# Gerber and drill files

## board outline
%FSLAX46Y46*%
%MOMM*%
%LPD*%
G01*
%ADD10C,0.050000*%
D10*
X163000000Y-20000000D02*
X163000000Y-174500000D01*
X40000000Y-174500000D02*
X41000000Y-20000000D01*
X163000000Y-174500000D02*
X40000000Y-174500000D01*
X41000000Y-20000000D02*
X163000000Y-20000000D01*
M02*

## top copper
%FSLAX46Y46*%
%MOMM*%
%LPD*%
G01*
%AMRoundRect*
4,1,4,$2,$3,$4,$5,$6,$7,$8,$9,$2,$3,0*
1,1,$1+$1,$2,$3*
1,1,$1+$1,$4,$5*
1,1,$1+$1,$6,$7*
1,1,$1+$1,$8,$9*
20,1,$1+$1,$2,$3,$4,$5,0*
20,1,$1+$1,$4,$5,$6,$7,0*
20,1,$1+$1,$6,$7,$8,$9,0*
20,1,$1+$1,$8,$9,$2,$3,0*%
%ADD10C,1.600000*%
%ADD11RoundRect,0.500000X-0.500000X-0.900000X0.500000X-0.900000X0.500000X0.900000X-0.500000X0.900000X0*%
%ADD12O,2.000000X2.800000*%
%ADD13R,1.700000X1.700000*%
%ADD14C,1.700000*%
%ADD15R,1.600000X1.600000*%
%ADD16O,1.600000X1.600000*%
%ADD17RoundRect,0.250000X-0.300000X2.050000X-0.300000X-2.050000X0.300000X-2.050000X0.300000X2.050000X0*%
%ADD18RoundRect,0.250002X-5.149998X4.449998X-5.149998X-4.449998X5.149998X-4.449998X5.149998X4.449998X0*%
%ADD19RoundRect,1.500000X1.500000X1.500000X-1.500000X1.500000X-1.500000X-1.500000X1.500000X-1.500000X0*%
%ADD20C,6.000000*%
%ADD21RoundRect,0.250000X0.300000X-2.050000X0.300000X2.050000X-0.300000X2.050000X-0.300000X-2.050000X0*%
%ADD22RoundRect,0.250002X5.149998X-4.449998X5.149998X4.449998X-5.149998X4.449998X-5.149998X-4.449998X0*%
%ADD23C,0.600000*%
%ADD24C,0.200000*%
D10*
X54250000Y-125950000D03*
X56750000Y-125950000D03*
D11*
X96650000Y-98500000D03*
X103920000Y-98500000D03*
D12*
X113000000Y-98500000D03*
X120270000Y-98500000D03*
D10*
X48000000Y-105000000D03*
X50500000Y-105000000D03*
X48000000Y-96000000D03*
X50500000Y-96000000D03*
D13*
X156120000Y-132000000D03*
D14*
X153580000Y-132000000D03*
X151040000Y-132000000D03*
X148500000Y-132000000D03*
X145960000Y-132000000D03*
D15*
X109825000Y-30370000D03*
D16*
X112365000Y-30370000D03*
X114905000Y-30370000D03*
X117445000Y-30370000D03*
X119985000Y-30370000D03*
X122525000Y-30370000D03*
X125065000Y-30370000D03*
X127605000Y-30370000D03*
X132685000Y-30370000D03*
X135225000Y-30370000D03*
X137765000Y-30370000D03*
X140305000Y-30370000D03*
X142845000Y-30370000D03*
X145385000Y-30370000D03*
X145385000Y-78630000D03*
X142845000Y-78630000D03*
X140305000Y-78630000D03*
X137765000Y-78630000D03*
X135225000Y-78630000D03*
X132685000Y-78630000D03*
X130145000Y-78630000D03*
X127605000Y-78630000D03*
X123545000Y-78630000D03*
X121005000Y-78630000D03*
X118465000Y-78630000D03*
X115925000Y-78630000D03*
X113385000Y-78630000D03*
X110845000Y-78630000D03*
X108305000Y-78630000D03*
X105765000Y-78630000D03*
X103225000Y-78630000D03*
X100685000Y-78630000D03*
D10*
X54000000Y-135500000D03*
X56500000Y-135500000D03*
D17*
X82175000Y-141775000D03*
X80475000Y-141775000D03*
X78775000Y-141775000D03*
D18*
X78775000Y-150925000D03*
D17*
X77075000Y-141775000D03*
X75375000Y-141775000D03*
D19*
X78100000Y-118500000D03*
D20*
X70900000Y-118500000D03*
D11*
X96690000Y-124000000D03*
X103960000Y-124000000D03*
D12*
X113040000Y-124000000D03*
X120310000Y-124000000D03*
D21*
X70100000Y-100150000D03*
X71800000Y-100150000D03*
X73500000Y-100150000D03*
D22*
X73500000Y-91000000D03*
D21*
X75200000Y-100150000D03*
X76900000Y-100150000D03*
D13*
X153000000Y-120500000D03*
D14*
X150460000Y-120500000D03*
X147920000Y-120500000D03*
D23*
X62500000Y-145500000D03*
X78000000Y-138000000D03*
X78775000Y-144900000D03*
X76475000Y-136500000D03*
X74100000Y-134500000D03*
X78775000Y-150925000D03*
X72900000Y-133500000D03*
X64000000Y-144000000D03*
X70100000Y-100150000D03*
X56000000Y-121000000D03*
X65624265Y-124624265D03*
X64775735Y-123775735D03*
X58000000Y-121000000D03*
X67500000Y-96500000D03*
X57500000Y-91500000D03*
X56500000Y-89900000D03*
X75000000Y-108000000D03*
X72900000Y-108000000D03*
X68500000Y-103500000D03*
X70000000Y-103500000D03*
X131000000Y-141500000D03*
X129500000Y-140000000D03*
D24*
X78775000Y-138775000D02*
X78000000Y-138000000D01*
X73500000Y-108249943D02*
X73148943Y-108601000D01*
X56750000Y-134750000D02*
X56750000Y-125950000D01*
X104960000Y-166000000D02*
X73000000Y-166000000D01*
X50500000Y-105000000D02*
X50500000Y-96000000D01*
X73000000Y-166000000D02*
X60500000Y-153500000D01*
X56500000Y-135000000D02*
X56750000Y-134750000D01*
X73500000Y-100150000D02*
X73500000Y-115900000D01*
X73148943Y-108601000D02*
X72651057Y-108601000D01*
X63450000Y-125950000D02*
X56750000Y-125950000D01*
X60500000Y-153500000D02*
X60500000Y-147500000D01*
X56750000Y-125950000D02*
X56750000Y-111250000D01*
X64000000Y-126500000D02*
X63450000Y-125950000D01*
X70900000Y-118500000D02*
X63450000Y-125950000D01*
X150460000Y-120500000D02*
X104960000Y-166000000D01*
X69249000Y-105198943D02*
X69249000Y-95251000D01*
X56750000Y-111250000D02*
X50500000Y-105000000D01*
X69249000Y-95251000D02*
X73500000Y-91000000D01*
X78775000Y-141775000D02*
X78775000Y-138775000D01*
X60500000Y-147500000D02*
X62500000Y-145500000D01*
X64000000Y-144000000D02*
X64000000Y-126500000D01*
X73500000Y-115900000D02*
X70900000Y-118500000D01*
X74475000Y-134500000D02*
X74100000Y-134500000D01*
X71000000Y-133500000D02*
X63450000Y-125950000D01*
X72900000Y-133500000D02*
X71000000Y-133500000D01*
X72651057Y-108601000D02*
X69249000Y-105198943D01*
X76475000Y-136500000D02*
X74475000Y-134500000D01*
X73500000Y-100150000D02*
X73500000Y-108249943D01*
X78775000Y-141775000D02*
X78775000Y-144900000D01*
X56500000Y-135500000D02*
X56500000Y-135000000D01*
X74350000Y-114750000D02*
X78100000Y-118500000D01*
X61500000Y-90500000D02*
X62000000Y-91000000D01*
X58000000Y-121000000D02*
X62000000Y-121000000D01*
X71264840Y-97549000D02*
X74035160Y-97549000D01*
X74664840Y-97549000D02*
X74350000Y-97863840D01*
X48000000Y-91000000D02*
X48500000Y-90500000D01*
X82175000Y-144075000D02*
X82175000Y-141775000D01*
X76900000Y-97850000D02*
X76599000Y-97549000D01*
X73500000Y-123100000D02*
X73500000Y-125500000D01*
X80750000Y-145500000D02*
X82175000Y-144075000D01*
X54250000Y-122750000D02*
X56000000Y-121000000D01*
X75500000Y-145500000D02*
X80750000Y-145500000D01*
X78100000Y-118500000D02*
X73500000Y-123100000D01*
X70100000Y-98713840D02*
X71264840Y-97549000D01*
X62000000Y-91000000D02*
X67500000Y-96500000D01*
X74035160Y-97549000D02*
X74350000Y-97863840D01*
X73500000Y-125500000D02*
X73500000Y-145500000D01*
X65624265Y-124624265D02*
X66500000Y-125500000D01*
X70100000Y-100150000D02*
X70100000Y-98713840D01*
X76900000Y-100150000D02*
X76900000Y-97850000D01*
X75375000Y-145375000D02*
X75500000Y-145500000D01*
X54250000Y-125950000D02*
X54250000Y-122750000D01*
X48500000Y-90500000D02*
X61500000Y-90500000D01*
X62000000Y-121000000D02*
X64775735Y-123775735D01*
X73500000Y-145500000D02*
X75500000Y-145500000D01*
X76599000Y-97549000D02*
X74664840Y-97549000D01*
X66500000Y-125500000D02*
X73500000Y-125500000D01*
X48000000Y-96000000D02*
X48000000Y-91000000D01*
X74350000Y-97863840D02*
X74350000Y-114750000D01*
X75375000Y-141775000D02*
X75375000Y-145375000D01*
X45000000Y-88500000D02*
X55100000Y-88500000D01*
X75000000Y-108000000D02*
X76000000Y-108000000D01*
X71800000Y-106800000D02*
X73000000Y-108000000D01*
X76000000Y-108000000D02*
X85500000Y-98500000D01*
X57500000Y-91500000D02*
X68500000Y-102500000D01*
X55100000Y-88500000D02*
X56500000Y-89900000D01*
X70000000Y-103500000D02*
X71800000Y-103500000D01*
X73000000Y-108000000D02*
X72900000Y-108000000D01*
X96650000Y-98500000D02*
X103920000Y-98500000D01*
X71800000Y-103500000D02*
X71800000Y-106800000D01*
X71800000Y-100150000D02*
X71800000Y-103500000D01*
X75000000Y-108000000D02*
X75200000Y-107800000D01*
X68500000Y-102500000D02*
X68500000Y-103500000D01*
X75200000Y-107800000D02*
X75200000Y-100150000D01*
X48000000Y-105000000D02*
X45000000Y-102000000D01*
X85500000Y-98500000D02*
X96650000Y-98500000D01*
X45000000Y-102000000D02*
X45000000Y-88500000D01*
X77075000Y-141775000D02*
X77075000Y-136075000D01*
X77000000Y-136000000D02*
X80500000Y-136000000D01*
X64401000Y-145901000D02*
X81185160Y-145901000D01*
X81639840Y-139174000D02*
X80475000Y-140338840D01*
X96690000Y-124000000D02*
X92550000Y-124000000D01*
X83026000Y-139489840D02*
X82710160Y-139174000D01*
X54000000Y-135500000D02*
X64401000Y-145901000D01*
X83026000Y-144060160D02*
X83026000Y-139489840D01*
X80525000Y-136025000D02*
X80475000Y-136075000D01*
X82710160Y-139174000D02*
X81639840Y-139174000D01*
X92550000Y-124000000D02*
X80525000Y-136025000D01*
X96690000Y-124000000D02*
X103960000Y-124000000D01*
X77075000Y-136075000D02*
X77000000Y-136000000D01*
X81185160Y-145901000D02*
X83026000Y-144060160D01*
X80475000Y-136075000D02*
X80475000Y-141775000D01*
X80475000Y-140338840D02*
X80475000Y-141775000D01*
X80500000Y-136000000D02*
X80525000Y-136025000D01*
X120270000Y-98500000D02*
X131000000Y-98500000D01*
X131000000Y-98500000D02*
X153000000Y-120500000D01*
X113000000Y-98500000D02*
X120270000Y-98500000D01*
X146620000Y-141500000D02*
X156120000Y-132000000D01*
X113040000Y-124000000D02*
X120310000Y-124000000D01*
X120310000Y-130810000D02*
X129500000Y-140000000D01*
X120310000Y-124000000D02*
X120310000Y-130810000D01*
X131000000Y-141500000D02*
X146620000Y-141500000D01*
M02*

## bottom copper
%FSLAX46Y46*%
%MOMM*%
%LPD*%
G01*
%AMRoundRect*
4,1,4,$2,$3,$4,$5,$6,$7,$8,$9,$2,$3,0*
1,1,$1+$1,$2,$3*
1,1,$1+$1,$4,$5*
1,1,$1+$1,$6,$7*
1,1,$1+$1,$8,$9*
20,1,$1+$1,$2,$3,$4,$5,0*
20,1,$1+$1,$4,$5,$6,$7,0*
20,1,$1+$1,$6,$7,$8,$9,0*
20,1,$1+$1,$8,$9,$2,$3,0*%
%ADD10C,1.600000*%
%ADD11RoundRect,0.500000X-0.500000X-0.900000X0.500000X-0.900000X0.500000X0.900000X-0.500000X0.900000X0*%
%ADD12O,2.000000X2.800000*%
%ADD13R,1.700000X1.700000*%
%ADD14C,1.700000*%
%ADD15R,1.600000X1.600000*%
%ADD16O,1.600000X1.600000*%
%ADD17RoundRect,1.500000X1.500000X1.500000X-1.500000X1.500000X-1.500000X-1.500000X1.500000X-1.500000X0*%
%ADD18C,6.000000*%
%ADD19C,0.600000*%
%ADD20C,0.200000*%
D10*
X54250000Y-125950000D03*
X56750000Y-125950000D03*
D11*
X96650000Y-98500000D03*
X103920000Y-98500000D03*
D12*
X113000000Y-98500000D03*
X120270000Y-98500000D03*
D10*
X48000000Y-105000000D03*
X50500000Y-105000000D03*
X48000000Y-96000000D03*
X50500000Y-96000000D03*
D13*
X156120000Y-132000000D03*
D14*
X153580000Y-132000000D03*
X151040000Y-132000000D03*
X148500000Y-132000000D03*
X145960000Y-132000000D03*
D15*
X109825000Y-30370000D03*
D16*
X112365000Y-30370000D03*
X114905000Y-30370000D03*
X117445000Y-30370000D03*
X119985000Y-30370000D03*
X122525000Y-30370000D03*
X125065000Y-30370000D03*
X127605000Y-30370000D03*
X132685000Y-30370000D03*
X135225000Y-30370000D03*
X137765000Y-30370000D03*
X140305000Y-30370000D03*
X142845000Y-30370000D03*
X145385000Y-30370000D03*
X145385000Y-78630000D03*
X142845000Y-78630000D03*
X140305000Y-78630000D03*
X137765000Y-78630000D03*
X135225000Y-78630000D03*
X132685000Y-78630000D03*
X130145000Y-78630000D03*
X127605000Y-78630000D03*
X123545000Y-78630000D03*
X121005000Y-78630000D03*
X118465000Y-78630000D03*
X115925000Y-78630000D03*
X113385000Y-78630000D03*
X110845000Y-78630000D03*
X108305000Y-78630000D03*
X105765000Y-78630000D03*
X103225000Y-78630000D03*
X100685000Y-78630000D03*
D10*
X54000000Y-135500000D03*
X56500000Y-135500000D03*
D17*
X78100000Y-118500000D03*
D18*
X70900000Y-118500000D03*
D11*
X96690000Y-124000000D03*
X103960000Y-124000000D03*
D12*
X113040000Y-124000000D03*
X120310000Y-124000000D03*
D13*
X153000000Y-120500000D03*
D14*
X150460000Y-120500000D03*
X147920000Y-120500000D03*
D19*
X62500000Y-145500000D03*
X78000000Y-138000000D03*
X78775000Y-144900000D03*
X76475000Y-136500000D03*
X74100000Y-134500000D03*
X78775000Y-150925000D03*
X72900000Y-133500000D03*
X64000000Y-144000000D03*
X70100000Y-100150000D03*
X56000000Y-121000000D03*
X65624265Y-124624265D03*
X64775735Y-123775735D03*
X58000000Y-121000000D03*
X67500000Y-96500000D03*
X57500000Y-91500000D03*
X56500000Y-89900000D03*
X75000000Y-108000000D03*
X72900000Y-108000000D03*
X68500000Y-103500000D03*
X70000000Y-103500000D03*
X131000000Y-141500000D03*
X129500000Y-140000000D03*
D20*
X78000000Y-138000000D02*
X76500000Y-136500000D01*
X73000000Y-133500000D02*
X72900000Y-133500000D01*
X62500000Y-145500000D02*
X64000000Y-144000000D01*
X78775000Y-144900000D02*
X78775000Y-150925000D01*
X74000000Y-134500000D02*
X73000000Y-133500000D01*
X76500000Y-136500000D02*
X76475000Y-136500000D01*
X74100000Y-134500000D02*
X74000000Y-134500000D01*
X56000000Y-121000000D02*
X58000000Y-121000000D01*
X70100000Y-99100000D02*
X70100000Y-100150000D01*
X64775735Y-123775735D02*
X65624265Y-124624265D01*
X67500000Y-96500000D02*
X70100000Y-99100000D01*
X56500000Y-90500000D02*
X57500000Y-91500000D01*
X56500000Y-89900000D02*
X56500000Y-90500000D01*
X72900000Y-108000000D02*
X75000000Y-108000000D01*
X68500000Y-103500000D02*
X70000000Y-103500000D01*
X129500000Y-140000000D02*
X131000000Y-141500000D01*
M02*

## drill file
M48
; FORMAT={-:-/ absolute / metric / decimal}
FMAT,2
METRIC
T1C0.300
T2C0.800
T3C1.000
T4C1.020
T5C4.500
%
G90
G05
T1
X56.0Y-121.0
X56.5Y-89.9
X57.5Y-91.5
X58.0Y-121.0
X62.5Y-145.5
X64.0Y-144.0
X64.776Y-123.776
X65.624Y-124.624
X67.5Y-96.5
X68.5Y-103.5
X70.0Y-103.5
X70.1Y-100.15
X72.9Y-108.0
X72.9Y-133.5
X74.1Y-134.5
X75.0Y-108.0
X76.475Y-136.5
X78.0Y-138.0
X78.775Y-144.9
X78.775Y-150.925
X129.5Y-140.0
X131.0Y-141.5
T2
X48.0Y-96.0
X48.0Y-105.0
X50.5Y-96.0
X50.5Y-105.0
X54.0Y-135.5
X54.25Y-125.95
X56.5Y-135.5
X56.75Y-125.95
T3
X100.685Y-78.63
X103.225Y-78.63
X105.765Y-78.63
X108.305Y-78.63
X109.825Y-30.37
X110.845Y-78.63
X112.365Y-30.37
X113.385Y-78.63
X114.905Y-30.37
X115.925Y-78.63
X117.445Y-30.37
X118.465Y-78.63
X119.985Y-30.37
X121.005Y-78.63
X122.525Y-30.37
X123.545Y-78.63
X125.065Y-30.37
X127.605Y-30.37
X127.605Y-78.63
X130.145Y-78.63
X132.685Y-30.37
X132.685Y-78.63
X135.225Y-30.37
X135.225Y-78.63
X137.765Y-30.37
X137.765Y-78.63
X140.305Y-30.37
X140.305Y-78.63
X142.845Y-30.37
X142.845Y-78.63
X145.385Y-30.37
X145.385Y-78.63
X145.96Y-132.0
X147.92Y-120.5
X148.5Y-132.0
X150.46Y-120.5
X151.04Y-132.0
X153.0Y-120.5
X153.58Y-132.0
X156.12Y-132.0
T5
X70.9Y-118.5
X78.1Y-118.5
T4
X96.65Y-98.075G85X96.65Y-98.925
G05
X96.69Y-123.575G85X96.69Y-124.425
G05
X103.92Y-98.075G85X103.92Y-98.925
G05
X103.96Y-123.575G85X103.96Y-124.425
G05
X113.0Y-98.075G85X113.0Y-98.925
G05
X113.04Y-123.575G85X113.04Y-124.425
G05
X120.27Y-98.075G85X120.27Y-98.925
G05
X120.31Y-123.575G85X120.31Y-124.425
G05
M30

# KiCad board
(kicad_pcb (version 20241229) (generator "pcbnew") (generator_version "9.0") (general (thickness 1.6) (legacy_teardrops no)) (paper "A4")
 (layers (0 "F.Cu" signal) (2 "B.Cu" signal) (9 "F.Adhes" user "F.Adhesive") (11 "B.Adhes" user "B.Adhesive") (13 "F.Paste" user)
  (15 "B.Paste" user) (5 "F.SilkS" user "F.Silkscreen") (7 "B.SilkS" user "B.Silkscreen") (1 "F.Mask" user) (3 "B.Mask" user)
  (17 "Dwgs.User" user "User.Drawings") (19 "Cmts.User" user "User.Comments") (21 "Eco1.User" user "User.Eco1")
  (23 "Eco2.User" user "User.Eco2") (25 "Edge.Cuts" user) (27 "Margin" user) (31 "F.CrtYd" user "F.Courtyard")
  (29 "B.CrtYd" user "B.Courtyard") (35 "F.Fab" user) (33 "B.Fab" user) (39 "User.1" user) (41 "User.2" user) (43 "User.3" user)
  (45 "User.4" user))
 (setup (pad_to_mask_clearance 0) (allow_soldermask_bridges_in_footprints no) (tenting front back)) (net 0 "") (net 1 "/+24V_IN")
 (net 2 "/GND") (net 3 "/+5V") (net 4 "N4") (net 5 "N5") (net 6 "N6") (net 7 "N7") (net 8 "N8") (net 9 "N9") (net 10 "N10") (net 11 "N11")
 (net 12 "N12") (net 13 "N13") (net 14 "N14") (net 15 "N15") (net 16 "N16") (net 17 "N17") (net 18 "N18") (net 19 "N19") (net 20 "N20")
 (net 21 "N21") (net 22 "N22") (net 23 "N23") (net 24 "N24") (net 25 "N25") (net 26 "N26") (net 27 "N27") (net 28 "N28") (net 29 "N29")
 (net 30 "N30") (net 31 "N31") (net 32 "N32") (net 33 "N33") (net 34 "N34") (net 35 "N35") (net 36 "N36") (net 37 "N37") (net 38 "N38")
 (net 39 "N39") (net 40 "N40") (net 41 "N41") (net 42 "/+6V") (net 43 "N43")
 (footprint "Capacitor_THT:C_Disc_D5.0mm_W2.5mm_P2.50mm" (layer "F.Cu") (at 54.25 125.95)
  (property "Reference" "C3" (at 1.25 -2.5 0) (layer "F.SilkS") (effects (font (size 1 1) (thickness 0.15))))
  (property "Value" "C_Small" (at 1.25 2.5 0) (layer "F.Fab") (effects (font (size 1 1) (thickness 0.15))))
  (pad "1" thru_hole circle (at 0 0) (size 1.6 1.6) (drill 0.8) (layers "*.Cu" "*.Mask") (remove_unused_layers no) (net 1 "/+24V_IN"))
  (pad "2" thru_hole circle (at 2.5 0) (size 1.6 1.6) (drill 0.8) (layers "*.Cu" "*.Mask") (remove_unused_layers no) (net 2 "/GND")))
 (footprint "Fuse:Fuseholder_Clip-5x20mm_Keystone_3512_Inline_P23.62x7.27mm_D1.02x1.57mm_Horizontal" (layer "F.Cu") (at 96.65 98.5)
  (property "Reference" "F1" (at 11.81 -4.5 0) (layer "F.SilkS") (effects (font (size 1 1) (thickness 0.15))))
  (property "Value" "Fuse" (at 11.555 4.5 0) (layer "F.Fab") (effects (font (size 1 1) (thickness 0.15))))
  (pad "1" thru_hole roundrect (at 0 0) (size 2 2.8) (drill oval 1.02 1.87) (layers "*.Cu" "*.Mask") (remove_unused_layers no)
   (roundrect_rratio 0.25) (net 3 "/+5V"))
  (pad "1" thru_hole roundrect (at 7.27 0) (size 2 2.8) (drill oval 1.02 1.87) (layers "*.Cu" "*.Mask") (remove_unused_layers no)
   (roundrect_rratio 0.25) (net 3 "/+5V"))
  (pad "2" thru_hole oval (at 16.35 0) (size 2 2.8) (drill oval 1.02 1.87) (layers "*.Cu" "*.Mask") (remove_unused_layers no) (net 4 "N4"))
  (pad "2" thru_hole oval (at 23.62 0) (size 2 2.8) (drill oval 1.02 1.87) (layers "*.Cu" "*.Mask") (remove_unused_layers no) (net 4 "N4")))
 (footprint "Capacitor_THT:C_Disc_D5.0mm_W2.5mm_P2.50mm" (layer "F.Cu") (at 48 105)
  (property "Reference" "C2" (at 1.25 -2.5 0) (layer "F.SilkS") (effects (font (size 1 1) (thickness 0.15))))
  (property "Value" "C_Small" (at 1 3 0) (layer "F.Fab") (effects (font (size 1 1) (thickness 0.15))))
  (pad "1" thru_hole circle (at 0 0) (size 1.6 1.6) (drill 0.8) (layers "*.Cu" "*.Mask") (remove_unused_layers no) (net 3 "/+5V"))
  (pad "2" thru_hole circle (at 2.5 0) (size 1.6 1.6) (drill 0.8) (layers "*.Cu" "*.Mask") (remove_unused_layers no) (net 2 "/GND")))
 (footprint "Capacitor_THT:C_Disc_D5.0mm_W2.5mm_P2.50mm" (layer "F.Cu") (at 48 96)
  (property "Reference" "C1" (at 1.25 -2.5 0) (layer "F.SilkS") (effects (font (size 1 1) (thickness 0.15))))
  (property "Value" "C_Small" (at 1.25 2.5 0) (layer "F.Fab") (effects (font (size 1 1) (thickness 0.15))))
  (pad "1" thru_hole circle (at 0 0) (size 1.6 1.6) (drill 0.8) (layers "*.Cu" "*.Mask") (remove_unused_layers no) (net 1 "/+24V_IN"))
  (pad "2" thru_hole circle (at 2.5 0) (size 1.6 1.6) (drill 0.8) (layers "*.Cu" "*.Mask") (remove_unused_layers no) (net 2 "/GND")))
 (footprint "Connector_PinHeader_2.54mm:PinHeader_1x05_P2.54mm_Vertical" (layer "F.Cu") (at 156.12 132 -90)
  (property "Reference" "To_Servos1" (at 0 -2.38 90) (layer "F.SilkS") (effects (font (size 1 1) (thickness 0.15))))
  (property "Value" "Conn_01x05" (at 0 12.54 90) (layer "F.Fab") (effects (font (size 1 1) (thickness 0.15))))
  (pad "1" thru_hole rect (at 0 0 270) (size 1.7 1.7) (drill 1) (layers "*.Cu" "*.Mask") (remove_unused_layers no) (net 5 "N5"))
  (pad "2" thru_hole circle (at 0 2.54 270) (size 1.7 1.7) (drill 1) (layers "*.Cu" "*.Mask") (remove_unused_layers no) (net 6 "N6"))
  (pad "3" thru_hole circle (at 0 5.08 270) (size 1.7 1.7) (drill 1) (layers "*.Cu" "*.Mask") (remove_unused_layers no) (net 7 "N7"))
  (pad "4" thru_hole circle (at 0 7.62 270) (size 1.7 1.7) (drill 1) (layers "*.Cu" "*.Mask") (remove_unused_layers no) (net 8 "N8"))
  (pad "5" thru_hole circle (at 0 10.16 270) (size 1.7 1.7) (drill 1) (layers "*.Cu" "*.Mask") (remove_unused_layers no) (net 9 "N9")))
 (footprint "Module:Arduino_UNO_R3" (layer "F.Cu") (at 109.825 30.37)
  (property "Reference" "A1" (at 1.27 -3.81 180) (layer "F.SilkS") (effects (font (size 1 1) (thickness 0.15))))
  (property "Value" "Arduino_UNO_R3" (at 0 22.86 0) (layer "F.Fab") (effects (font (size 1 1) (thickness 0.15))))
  (pad "1" thru_hole rect (at 0 0 90) (size 1.6 1.6) (drill 1) (layers "*.Cu" "*.Mask") (remove_unused_layers no) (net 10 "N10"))
  (pad "2" thru_hole oval (at 2.54 0 90) (size 1.6 1.6) (drill 1) (layers "*.Cu" "*.Mask") (remove_unused_layers no) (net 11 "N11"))
  (pad "3" thru_hole oval (at 5.08 0 90) (size 1.6 1.6) (drill 1) (layers "*.Cu" "*.Mask") (remove_unused_layers no) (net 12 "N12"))
  (pad "4" thru_hole oval (at 7.62 0 90) (size 1.6 1.6) (drill 1) (layers "*.Cu" "*.Mask") (remove_unused_layers no) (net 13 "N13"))
  (pad "5" thru_hole oval (at 10.16 0 90) (size 1.6 1.6) (drill 1) (layers "*.Cu" "*.Mask") (remove_unused_layers no) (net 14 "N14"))
  (pad "6" thru_hole oval (at 12.7 0 90) (size 1.6 1.6) (drill 1) (layers "*.Cu" "*.Mask") (remove_unused_layers no) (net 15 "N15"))
  (pad "7" thru_hole oval (at 15.24 0 90) (size 1.6 1.6) (drill 1) (layers "*.Cu" "*.Mask") (remove_unused_layers no) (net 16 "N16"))
  (pad "8" thru_hole oval (at 17.78 0 90) (size 1.6 1.6) (drill 1) (layers "*.Cu" "*.Mask") (remove_unused_layers no) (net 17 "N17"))
  (pad "9" thru_hole oval (at 22.86 0 90) (size 1.6 1.6) (drill 1) (layers "*.Cu" "*.Mask") (remove_unused_layers no) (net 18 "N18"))
  (pad "10" thru_hole oval (at 25.4 0 90) (size 1.6 1.6) (drill 1) (layers "*.Cu" "*.Mask") (remove_unused_layers no) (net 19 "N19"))
  (pad "11" thru_hole oval (at 27.94 0 90) (size 1.6 1.6) (drill 1) (layers "*.Cu" "*.Mask") (remove_unused_layers no) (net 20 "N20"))
  (pad "12" thru_hole oval (at 30.48 0 90) (size 1.6 1.6) (drill 1) (layers "*.Cu" "*.Mask") (remove_unused_layers no) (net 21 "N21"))
  (pad "13" thru_hole oval (at 33.02 0 90) (size 1.6 1.6) (drill 1) (layers "*.Cu" "*.Mask") (remove_unused_layers no) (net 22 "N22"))
  (pad "14" thru_hole oval (at 35.56 0 90) (size 1.6 1.6) (drill 1) (layers "*.Cu" "*.Mask") (remove_unused_layers no) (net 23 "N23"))
  (pad "15" thru_hole oval (at 35.56 48.26 90) (size 1.6 1.6) (drill 1) (layers "*.Cu" "*.Mask") (remove_unused_layers no) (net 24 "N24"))
  (pad "16" thru_hole oval (at 33.02 48.26 90) (size 1.6 1.6) (drill 1) (layers "*.Cu" "*.Mask") (remove_unused_layers no) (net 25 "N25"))
  (pad "17" thru_hole oval (at 30.48 48.26 90) (size 1.6 1.6) (drill 1) (layers "*.Cu" "*.Mask") (remove_unused_layers no) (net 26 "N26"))
  (pad "18" thru_hole oval (at 27.94 48.26 90) (size 1.6 1.6) (drill 1) (layers "*.Cu" "*.Mask") (remove_unused_layers no) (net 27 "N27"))
  (pad "19" thru_hole oval (at 25.4 48.26 90) (size 1.6 1.6) (drill 1) (layers "*.Cu" "*.Mask") (remove_unused_layers no) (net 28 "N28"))
  (pad "20" thru_hole oval (at 22.86 48.26 90) (size 1.6 1.6) (drill 1) (layers "*.Cu" "*.Mask") (remove_unused_layers no) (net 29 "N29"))
  (pad "21" thru_hole oval (at 20.32 48.26 90) (size 1.6 1.6) (drill 1) (layers "*.Cu" "*.Mask") (remove_unused_layers no) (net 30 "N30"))
  (pad "22" thru_hole oval (at 17.78 48.26 90) (size 1.6 1.6) (drill 1) (layers "*.Cu" "*.Mask") (remove_unused_layers no) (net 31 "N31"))
  (pad "23" thru_hole oval (at 13.72 48.26 90) (size 1.6 1.6) (drill 1) (layers "*.Cu" "*.Mask") (remove_unused_layers no) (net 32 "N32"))
  (pad "24" thru_hole oval (at 11.18 48.26 90) (size 1.6 1.6) (drill 1) (layers "*.Cu" "*.Mask") (remove_unused_layers no) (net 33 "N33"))
  (pad "25" thru_hole oval (at 8.64 48.26 90) (size 1.6 1.6) (drill 1) (layers "*.Cu" "*.Mask") (remove_unused_layers no) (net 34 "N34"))
  (pad "26" thru_hole oval (at 6.1 48.26 90) (size 1.6 1.6) (drill 1) (layers "*.Cu" "*.Mask") (remove_unused_layers no) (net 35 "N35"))
  (pad "27" thru_hole oval (at 3.56 48.26 90) (size 1.6 1.6) (drill 1) (layers "*.Cu" "*.Mask") (remove_unused_layers no) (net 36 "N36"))
  (pad "28" thru_hole oval (at 1.02 48.26 90) (size 1.6 1.6) (drill 1) (layers "*.Cu" "*.Mask") (remove_unused_layers no) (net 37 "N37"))
  (pad "29" thru_hole oval (at -1.52 48.26 90) (size 1.6 1.6) (drill 1) (layers "*.Cu" "*.Mask") (remove_unused_layers no) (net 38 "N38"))
  (pad "30" thru_hole oval (at -4.06 48.26 90) (size 1.6 1.6) (drill 1) (layers "*.Cu" "*.Mask") (remove_unused_layers no) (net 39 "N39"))
  (pad "31" thru_hole oval (at -6.6 48.26 90) (size 1.6 1.6) (drill 1) (layers "*.Cu" "*.Mask") (remove_unused_layers no) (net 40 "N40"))
  (pad "32" thru_hole oval (at -9.14 48.26 90) (size 1.6 1.6) (drill 1) (layers "*.Cu" "*.Mask") (remove_unused_layers no) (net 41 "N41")))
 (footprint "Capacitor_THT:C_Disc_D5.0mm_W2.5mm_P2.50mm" (layer "F.Cu") (at 54 135.5)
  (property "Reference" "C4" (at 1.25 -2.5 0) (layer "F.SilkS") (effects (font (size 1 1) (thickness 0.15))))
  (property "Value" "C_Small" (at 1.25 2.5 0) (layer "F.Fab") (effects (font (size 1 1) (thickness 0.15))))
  (pad "1" thru_hole circle (at 0 0) (size 1.6 1.6) (drill 0.8) (layers "*.Cu" "*.Mask") (remove_unused_layers no) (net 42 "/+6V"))
  (pad "2" thru_hole circle (at 2.5 0) (size 1.6 1.6) (drill 0.8) (layers "*.Cu" "*.Mask") (remove_unused_layers no) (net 2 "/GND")))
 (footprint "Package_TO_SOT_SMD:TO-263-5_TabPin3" (layer "F.Cu") (at 78.775 149.425 -90)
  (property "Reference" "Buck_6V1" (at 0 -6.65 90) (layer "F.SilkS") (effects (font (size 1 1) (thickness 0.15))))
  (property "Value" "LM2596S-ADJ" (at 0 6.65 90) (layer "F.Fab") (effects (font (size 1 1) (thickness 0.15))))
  (pad "" smd roundrect (at -0.925 -2.775 270) (size 4.55 5.25) (layers "F.Paste") (roundrect_rratio 0.054945))
  (pad "" smd roundrect (at -0.925 2.775 270) (size 4.55 5.25) (layers "F.Paste") (roundrect_rratio 0.054945))
  (pad "" smd roundrect (at 3.925 -2.775 270) (size 4.55 5.25) (layers "F.Paste") (roundrect_rratio 0.054945))
  (pad "" smd roundrect (at 3.925 2.775 270) (size 4.55 5.25) (layers "F.Paste") (roundrect_rratio 0.054945))
  (pad "1" smd roundrect (at -7.65 -3.4 270) (size 4.6 1.1) (layers "F.Cu" "F.Mask" "F.Paste") (roundrect_rratio 0.227273)
   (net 1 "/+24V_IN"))
  (pad "2" smd roundrect (at -7.65 -1.7 270) (size 4.6 1.1) (layers "F.Cu" "F.Mask" "F.Paste") (roundrect_rratio 0.227273) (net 42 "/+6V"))
  (pad "3" smd roundrect (at -7.65 0 270) (size 4.6 1.1) (layers "F.Cu" "F.Mask" "F.Paste") (roundrect_rratio 0.227273) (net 2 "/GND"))
  (pad "3" smd roundrect (at 1.5 0 270) (size 9.4 10.8) (layers "F.Cu" "F.Mask") (roundrect_rratio 0.026596) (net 2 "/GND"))
  (pad "4" smd roundrect (at -7.65 1.7 270) (size 4.6 1.1) (layers "F.Cu" "F.Mask" "F.Paste") (roundrect_rratio 0.227273) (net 42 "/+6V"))
  (pad "5" smd roundrect (at -7.65 3.4 270) (size 4.6 1.1) (layers "F.Cu" "F.Mask" "F.Paste") (roundrect_rratio 0.227273) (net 1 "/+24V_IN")))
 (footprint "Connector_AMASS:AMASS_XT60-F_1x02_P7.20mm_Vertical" (layer "F.Cu") (at 78.1 118.5 180)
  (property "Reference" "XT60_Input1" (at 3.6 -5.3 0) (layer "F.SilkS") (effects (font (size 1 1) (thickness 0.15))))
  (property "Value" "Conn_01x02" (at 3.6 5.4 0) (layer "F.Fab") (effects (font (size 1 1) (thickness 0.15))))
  (pad "1" thru_hole roundrect (at 0 0 180) (size 6 6) (drill 4.5) (layers "*.Cu" "*.Mask") (remove_unused_layers no)
   (roundrect_rratio 0.25) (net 1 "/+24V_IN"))
  (pad "2" thru_hole circle (at 7.2 0 180) (size 6 6) (drill 4.5) (layers "*.Cu" "*.Mask") (remove_unused_layers no) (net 2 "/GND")))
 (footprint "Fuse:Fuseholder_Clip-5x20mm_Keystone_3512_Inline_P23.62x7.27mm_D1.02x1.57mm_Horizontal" (layer "F.Cu") (at 96.69 124)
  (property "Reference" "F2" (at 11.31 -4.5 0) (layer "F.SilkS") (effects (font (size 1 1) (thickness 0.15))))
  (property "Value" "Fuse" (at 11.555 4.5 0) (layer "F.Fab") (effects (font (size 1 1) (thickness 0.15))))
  (pad "1" thru_hole roundrect (at 0 0) (size 2 2.8) (drill oval 1.02 1.87) (layers "*.Cu" "*.Mask") (remove_unused_layers no)
   (roundrect_rratio 0.25) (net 42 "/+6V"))
  (pad "1" thru_hole roundrect (at 7.27 0) (size 2 2.8) (drill oval 1.02 1.87) (layers "*.Cu" "*.Mask") (remove_unused_layers no)
   (roundrect_rratio 0.25) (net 42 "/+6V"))
  (pad "2" thru_hole oval (at 16.35 0) (size 2 2.8) (drill oval 1.02 1.87) (layers "*.Cu" "*.Mask") (remove_unused_layers no) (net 5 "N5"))
  (pad "2" thru_hole oval (at 23.62 0) (size 2 2.8) (drill oval 1.02 1.87) (layers "*.Cu" "*.Mask") (remove_unused_layers no) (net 5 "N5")))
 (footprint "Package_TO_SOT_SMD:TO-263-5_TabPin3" (layer "F.Cu") (at 73.5 92.5 90)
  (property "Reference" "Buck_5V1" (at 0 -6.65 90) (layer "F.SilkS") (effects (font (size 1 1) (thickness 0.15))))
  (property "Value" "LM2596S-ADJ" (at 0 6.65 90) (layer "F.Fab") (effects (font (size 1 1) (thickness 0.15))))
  (pad "" smd roundrect (at -0.925 -2.775 90) (size 4.55 5.25) (layers "F.Paste") (roundrect_rratio 0.054945))
  (pad "" smd roundrect (at -0.925 2.775 90) (size 4.55 5.25) (layers "F.Paste") (roundrect_rratio 0.054945))
  (pad "" smd roundrect (at 3.925 -2.775 90) (size 4.55 5.25) (layers "F.Paste") (roundrect_rratio 0.054945))
  (pad "" smd roundrect (at 3.925 2.775 90) (size 4.55 5.25) (layers "F.Paste") (roundrect_rratio 0.054945))
  (pad "1" smd roundrect (at -7.65 -3.4 90) (size 4.6 1.1) (layers "F.Cu" "F.Mask" "F.Paste") (roundrect_rratio 0.227273) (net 1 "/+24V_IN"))
  (pad "2" smd roundrect (at -7.65 -1.7 90) (size 4.6 1.1) (layers "F.Cu" "F.Mask" "F.Paste") (roundrect_rratio 0.227273) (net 3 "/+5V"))
  (pad "3" smd roundrect (at -7.65 0 90) (size 4.6 1.1) (layers "F.Cu" "F.Mask" "F.Paste") (roundrect_rratio 0.227273) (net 2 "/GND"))
  (pad "3" smd roundrect (at 1.5 0 90) (size 9.4 10.8) (layers "F.Cu" "F.Mask") (roundrect_rratio 0.026596) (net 2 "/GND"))
  (pad "4" smd roundrect (at -7.65 1.7 90) (size 4.6 1.1) (layers "F.Cu" "F.Mask" "F.Paste") (roundrect_rratio 0.227273) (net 3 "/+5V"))
  (pad "5" smd roundrect (at -7.65 3.4 90) (size 4.6 1.1) (layers "F.Cu" "F.Mask" "F.Paste") (roundrect_rratio 0.227273) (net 1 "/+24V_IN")))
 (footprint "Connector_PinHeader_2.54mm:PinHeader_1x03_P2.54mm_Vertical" (layer "F.Cu") (at 153 120.5 -90)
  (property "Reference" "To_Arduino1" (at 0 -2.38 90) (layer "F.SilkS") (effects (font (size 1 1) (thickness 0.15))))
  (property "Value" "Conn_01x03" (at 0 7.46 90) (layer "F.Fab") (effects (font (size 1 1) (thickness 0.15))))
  (pad "1" thru_hole rect (at 0 0 270) (size 1.7 1.7) (drill 1) (layers "*.Cu" "*.Mask") (remove_unused_layers no) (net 4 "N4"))
  (pad "2" thru_hole circle (at 0 2.54 270) (size 1.7 1.7) (drill 1) (layers "*.Cu" "*.Mask") (remove_unused_layers no) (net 2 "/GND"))
  (pad "3" thru_hole circle (at 0 5.08 270) (size 1.7 1.7) (drill 1) (layers "*.Cu" "*.Mask") (remove_unused_layers no) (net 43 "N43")))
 (gr_line (start 163 20) (end 163 174.5) (stroke (width 0.05) (type default)) (layer "Edge.Cuts"))
 (gr_line (start 40 174.5) (end 41 20) (stroke (width 0.05) (type default)) (layer "Edge.Cuts"))
 (gr_line (start 163 174.5) (end 40 174.5) (stroke (width 0.05) (type default)) (layer "Edge.Cuts"))
 (gr_line (start 41 20) (end 163 20) (stroke (width 0.05) (type default)) (layer "Edge.Cuts"))
 (segment (start 78.775 138.775) (end 78 138) (width 0.2) (layer "F.Cu") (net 2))
 (segment (start 73.5 108.249943) (end 73.148943 108.601) (width 0.2) (layer "F.Cu") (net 2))
 (segment (start 56.75 134.75) (end 56.75 125.95) (width 0.2) (layer "F.Cu") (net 2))
 (segment (start 104.96 166) (end 73 166) (width 0.2) (layer "F.Cu") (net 2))
 (segment (start 50.5 105) (end 50.5 96) (width 0.2) (layer "F.Cu") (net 2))
 (segment (start 73 166) (end 60.5 153.5) (width 0.2) (layer "F.Cu") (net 2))
 (segment (start 56.5 135) (end 56.75 134.75) (width 0.2) (layer "F.Cu") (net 2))
 (segment (start 73.5 100.15) (end 73.5 115.9) (width 0.2) (layer "F.Cu") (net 2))
 (segment (start 73.148943 108.601) (end 72.651057 108.601) (width 0.2) (layer "F.Cu") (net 2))
 (segment (start 63.45 125.95) (end 56.75 125.95) (width 0.2) (layer "F.Cu") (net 2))
 (segment (start 60.5 153.5) (end 60.5 147.5) (width 0.2) (layer "F.Cu") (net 2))
 (segment (start 56.75 125.95) (end 56.75 111.25) (width 0.2) (layer "F.Cu") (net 2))
 (segment (start 64 126.5) (end 63.45 125.95) (width 0.2) (layer "F.Cu") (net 2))
 (segment (start 70.9 118.5) (end 63.45 125.95) (width 0.2) (layer "F.Cu") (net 2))
 (segment (start 150.46 120.5) (end 104.96 166) (width 0.2) (layer "F.Cu") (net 2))
 (segment (start 69.249 105.198943) (end 69.249 95.251) (width 0.2) (layer "F.Cu") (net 2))
 (segment (start 56.75 111.25) (end 50.5 105) (width 0.2) (layer "F.Cu") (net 2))
 (segment (start 69.249 95.251) (end 73.5 91) (width 0.2) (layer "F.Cu") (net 2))
 (segment (start 78.775 141.775) (end 78.775 138.775) (width 0.2) (layer "F.Cu") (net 2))
 (segment (start 60.5 147.5) (end 62.5 145.5) (width 0.2) (layer "F.Cu") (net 2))
 (segment (start 64 144) (end 64 126.5) (width 0.2) (layer "F.Cu") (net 2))
 (segment (start 73.5 115.9) (end 70.9 118.5) (width 0.2) (layer "F.Cu") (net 2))
 (segment (start 74.475 134.5) (end 74.1 134.5) (width 0.2) (layer "F.Cu") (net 2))
 (segment (start 71 133.5) (end 63.45 125.95) (width 0.2) (layer "F.Cu") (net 2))
 (segment (start 72.9 133.5) (end 71 133.5) (width 0.2) (layer "F.Cu") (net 2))
 (segment (start 72.651057 108.601) (end 69.249 105.198943) (width 0.2) (layer "F.Cu") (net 2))
 (segment (start 76.475 136.5) (end 74.475 134.5) (width 0.2) (layer "F.Cu") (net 2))
 (segment (start 73.5 100.15) (end 73.5 108.249943) (width 0.2) (layer "F.Cu") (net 2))
 (segment (start 78.775 141.775) (end 78.775 144.9) (width 0.2) (layer "F.Cu") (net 2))
 (segment (start 56.5 135.5) (end 56.5 135) (width 0.2) (layer "F.Cu") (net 2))
 (via (at 62.5 145.5) (size 0.6) (drill 0.3) (layers "F.Cu" "B.Cu") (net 2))
 (via (at 78 138) (size 0.6) (drill 0.3) (layers "F.Cu" "B.Cu") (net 2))
 (via (at 78.775 144.9) (size 0.6) (drill 0.3) (layers "F.Cu" "B.Cu") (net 2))
 (via (at 76.475 136.5) (size 0.6) (drill 0.3) (layers "F.Cu" "B.Cu") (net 2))
 (via (at 74.1 134.5) (size 0.6) (drill 0.3) (layers "F.Cu" "B.Cu") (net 2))
 (via (at 78.775 150.925) (size 0.6) (drill 0.3) (layers "F.Cu" "B.Cu") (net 2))
 (via (at 72.9 133.5) (size 0.6) (drill 0.3) (layers "F.Cu" "B.Cu") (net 2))
 (via (at 64 144) (size 0.6) (drill 0.3) (layers "F.Cu" "B.Cu") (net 2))
 (segment (start 78 138) (end 76.5 136.5) (width 0.2) (layer "B.Cu") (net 2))
 (segment (start 73 133.5) (end 72.9 133.5) (width 0.2) (layer "B.Cu") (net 2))
 (segment (start 62.5 145.5) (end 64 144) (width 0.2) (layer "B.Cu") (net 2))
 (segment (start 78.775 144.9) (end 78.775 150.925) (width 0.2) (layer "B.Cu") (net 2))
 (segment (start 74 134.5) (end 73 133.5) (width 0.2) (layer "B.Cu") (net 2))
 (segment (start 76.5 136.5) (end 76.475 136.5) (width 0.2) (layer "B.Cu") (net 2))
 (segment (start 74.1 134.5) (end 74 134.5) (width 0.2) (layer "B.Cu") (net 2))
 (segment (start 74.35 114.75) (end 78.1 118.5) (width 0.2) (layer "F.Cu") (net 1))
 (segment (start 61.5 90.5) (end 62 91) (width 0.2) (layer "F.Cu") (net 1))
 (segment (start 58 121) (end 62 121) (width 0.2) (layer "F.Cu") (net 1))
 (segment (start 71.26484 97.549) (end 74.03516 97.549) (width 0.2) (layer "F.Cu") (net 1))
 (segment (start 74.66484 97.549) (end 74.35 97.86384) (width 0.2) (layer "F.Cu") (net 1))
 (segment (start 48 91) (end 48.5 90.5) (width 0.2) (layer "F.Cu") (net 1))
 (segment (start 82.175 144.075) (end 82.175 141.775) (width 0.2) (layer "F.Cu") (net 1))
 (segment (start 76.9 97.85) (end 76.599 97.549) (width 0.2) (layer "F.Cu") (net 1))
 (segment (start 73.5 123.1) (end 73.5 125.5) (width 0.2) (layer "F.Cu") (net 1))
 (segment (start 80.75 145.5) (end 82.175 144.075) (width 0.2) (layer "F.Cu") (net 1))
 (segment (start 54.25 122.75) (end 56 121) (width 0.2) (layer "F.Cu") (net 1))
 (segment (start 75.5 145.5) (end 80.75 145.5) (width 0.2) (layer "F.Cu") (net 1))
 (segment (start 78.1 118.5) (end 73.5 123.1) (width 0.2) (layer "F.Cu") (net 1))
 (segment (start 70.1 98.71384) (end 71.26484 97.549) (width 0.2) (layer "F.Cu") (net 1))
 (segment (start 62 91) (end 67.5 96.5) (width 0.2) (layer "F.Cu") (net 1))
 (segment (start 74.03516 97.549) (end 74.35 97.86384) (width 0.2) (layer "F.Cu") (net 1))
 (segment (start 73.5 125.5) (end 73.5 145.5) (width 0.2) (layer "F.Cu") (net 1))
 (segment (start 65.624265 124.624265) (end 66.5 125.5) (width 0.2) (layer "F.Cu") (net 1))
 (segment (start 70.1 100.15) (end 70.1 98.71384) (width 0.2) (layer "F.Cu") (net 1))
 (segment (start 76.9 100.15) (end 76.9 97.85) (width 0.2) (layer "F.Cu") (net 1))
 (segment (start 75.375 145.375) (end 75.5 145.5) (width 0.2) (layer "F.Cu") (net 1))
 (segment (start 54.25 125.95) (end 54.25 122.75) (width 0.2) (layer "F.Cu") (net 1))
 (segment (start 48.5 90.5) (end 61.5 90.5) (width 0.2) (layer "F.Cu") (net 1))
 (segment (start 62 121) (end 64.775735 123.775735) (width 0.2) (layer "F.Cu") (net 1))
 (segment (start 73.5 145.5) (end 75.5 145.5) (width 0.2) (layer "F.Cu") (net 1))
 (segment (start 76.599 97.549) (end 74.66484 97.549) (width 0.2) (layer "F.Cu") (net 1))
 (segment (start 66.5 125.5) (end 73.5 125.5) (width 0.2) (layer "F.Cu") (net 1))
 (segment (start 48 96) (end 48 91) (width 0.2) (layer "F.Cu") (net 1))
 (segment (start 74.35 97.86384) (end 74.35 114.75) (width 0.2) (layer "F.Cu") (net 1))
 (segment (start 75.375 141.775) (end 75.375 145.375) (width 0.2) (layer "F.Cu") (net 1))
 (via (at 70.1 100.15) (size 0.6) (drill 0.3) (layers "F.Cu" "B.Cu") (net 1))
 (via (at 56 121) (size 0.6) (drill 0.3) (layers "F.Cu" "B.Cu") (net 1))
 (via (at 65.624265 124.624265) (size 0.6) (drill 0.3) (layers "F.Cu" "B.Cu") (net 1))
 (via (at 64.775735 123.775735) (size 0.6) (drill 0.3) (layers "F.Cu" "B.Cu") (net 1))
 (via (at 58 121) (size 0.6) (drill 0.3) (layers "F.Cu" "B.Cu") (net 1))
 (via (at 67.5 96.5) (size 0.6) (drill 0.3) (layers "F.Cu" "B.Cu") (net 1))
 (segment (start 56 121) (end 58 121) (width 0.2) (layer "B.Cu") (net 1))
 (segment (start 70.1 99.1) (end 70.1 100.15) (width 0.2) (layer "B.Cu") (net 1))
 (segment (start 64.775735 123.775735) (end 65.624265 124.624265) (width 0.2) (layer "B.Cu") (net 1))
 (segment (start 67.5 96.5) (end 70.1 99.1) (width 0.2) (layer "B.Cu") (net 1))
 (segment (start 45 88.5) (end 55.1 88.5) (width 0.2) (layer "F.Cu") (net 3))
 (segment (start 75 108) (end 76 108) (width 0.2) (layer "F.Cu") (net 3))
 (segment (start 71.8 106.8) (end 73 108) (width 0.2) (layer "F.Cu") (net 3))
 (segment (start 76 108) (end 85.5 98.5) (width 0.2) (layer "F.Cu") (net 3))
 (segment (start 57.5 91.5) (end 68.5 102.5) (width 0.2) (layer "F.Cu") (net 3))
 (segment (start 55.1 88.5) (end 56.5 89.9) (width 0.2) (layer "F.Cu") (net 3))
 (segment (start 70 103.5) (end 71.8 103.5) (width 0.2) (layer "F.Cu") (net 3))
 (segment (start 73 108) (end 72.9 108) (width 0.2) (layer "F.Cu") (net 3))
 (segment (start 96.65 98.5) (end 103.92 98.5) (width 0.2) (layer "F.Cu") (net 3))
 (segment (start 71.8 103.5) (end 71.8 106.8) (width 0.2) (layer "F.Cu") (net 3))
 (segment (start 71.8 100.15) (end 71.8 103.5) (width 0.2) (layer "F.Cu") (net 3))
 (segment (start 75 108) (end 75.2 107.8) (width 0.2) (layer "F.Cu") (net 3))
 (segment (start 68.5 102.5) (end 68.5 103.5) (width 0.2) (layer "F.Cu") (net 3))
 (segment (start 75.2 107.8) (end 75.2 100.15) (width 0.2) (layer "F.Cu") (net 3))
 (segment (start 48 105) (end 45 102) (width 0.2) (layer "F.Cu") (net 3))
 (segment (start 85.5 98.5) (end 96.65 98.5) (width 0.2) (layer "F.Cu") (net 3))
 (segment (start 45 102) (end 45 88.5) (width 0.2) (layer "F.Cu") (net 3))
 (via (at 57.5 91.5) (size 0.6) (drill 0.3) (layers "F.Cu" "B.Cu") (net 3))
 (via (at 56.5 89.9) (size 0.6) (drill 0.3) (layers "F.Cu" "B.Cu") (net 3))
 (via (at 75 108) (size 0.6) (drill 0.3) (layers "F.Cu" "B.Cu") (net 3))
 (via (at 72.9 108) (size 0.6) (drill 0.3) (layers "F.Cu" "B.Cu") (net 3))
 (via (at 68.5 103.5) (size 0.6) (drill 0.3) (layers "F.Cu" "B.Cu") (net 3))
 (via (at 70 103.5) (size 0.6) (drill 0.3) (layers "F.Cu" "B.Cu") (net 3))
 (segment (start 56.5 90.5) (end 57.5 91.5) (width 0.2) (layer "B.Cu") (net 3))
 (segment (start 56.5 89.9) (end 56.5 90.5) (width 0.2) (layer "B.Cu") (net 3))
 (segment (start 72.9 108) (end 75 108) (width 0.2) (layer "B.Cu") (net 3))
 (segment (start 68.5 103.5) (end 70 103.5) (width 0.2) (layer "B.Cu") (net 3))
 (segment (start 77.075 141.775) (end 77.075 136.075) (width 0.2) (layer "F.Cu") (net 42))
 (segment (start 77 136) (end 80.5 136) (width 0.2) (layer "F.Cu") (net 42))
 (segment (start 64.401 145.901) (end 81.18516 145.901) (width 0.2) (layer "F.Cu") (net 42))
 (segment (start 81.63984 139.174) (end 80.475 140.33884) (width 0.2) (layer "F.Cu") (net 42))
 (segment (start 96.69 124) (end 92.55 124) (width 0.2) (layer "F.Cu") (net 42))
 (segment (start 83.026 139.48984) (end 82.71016 139.174) (width 0.2) (layer "F.Cu") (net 42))
 (segment (start 54 135.5) (end 64.401 145.901) (width 0.2) (layer "F.Cu") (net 42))
 (segment (start 83.026 144.06016) (end 83.026 139.48984) (width 0.2) (layer "F.Cu") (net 42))
 (segment (start 80.525 136.025) (end 80.475 136.075) (width 0.2) (layer "F.Cu") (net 42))
 (segment (start 82.71016 139.174) (end 81.63984 139.174) (width 0.2) (layer "F.Cu") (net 42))
 (segment (start 92.55 124) (end 80.525 136.025) (width 0.2) (layer "F.Cu") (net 42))
 (segment (start 96.69 124) (end 103.96 124) (width 0.2) (layer "F.Cu") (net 42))
 (segment (start 77.075 136.075) (end 77 136) (width 0.2) (layer "F.Cu") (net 42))
 (segment (start 81.18516 145.901) (end 83.026 144.06016) (width 0.2) (layer "F.Cu") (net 42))
 (segment (start 80.475 136.075) (end 80.475 141.775) (width 0.2) (layer "F.Cu") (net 42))
 (segment (start 80.475 140.33884) (end 80.475 141.775) (width 0.2) (layer "F.Cu") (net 42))
 (segment (start 80.5 136) (end 80.525 136.025) (width 0.2) (layer "F.Cu") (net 42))
 (segment (start 120.27 98.5) (end 131 98.5) (width 0.2) (layer "F.Cu") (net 4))
 (segment (start 131 98.5) (end 153 120.5) (width 0.2) (layer "F.Cu") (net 4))
 (segment (start 113 98.5) (end 120.27 98.5) (width 0.2) (layer "F.Cu") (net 4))
 (segment (start 146.62 141.5) (end 156.12 132) (width 0.2) (layer "F.Cu") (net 5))
 (segment (start 113.04 124) (end 120.31 124) (width 0.2) (layer "F.Cu") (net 5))
 (segment (start 120.31 130.81) (end 129.5 140) (width 0.2) (layer "F.Cu") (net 5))
 (segment (start 120.31 124) (end 120.31 130.81) (width 0.2) (layer "F.Cu") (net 5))
 (segment (start 131 141.5) (end 146.62 141.5) (width 0.2) (layer "F.Cu") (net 5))
 (via (at 131 141.5) (size 0.6) (drill 0.3) (layers "F.Cu" "B.Cu") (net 5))
 (via (at 129.5 140) (size 0.6) (drill 0.3) (layers "F.Cu" "B.Cu") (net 5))
 (segment (start 129.5 140) (end 131 141.5) (width 0.2) (layer "B.Cu") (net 5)))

